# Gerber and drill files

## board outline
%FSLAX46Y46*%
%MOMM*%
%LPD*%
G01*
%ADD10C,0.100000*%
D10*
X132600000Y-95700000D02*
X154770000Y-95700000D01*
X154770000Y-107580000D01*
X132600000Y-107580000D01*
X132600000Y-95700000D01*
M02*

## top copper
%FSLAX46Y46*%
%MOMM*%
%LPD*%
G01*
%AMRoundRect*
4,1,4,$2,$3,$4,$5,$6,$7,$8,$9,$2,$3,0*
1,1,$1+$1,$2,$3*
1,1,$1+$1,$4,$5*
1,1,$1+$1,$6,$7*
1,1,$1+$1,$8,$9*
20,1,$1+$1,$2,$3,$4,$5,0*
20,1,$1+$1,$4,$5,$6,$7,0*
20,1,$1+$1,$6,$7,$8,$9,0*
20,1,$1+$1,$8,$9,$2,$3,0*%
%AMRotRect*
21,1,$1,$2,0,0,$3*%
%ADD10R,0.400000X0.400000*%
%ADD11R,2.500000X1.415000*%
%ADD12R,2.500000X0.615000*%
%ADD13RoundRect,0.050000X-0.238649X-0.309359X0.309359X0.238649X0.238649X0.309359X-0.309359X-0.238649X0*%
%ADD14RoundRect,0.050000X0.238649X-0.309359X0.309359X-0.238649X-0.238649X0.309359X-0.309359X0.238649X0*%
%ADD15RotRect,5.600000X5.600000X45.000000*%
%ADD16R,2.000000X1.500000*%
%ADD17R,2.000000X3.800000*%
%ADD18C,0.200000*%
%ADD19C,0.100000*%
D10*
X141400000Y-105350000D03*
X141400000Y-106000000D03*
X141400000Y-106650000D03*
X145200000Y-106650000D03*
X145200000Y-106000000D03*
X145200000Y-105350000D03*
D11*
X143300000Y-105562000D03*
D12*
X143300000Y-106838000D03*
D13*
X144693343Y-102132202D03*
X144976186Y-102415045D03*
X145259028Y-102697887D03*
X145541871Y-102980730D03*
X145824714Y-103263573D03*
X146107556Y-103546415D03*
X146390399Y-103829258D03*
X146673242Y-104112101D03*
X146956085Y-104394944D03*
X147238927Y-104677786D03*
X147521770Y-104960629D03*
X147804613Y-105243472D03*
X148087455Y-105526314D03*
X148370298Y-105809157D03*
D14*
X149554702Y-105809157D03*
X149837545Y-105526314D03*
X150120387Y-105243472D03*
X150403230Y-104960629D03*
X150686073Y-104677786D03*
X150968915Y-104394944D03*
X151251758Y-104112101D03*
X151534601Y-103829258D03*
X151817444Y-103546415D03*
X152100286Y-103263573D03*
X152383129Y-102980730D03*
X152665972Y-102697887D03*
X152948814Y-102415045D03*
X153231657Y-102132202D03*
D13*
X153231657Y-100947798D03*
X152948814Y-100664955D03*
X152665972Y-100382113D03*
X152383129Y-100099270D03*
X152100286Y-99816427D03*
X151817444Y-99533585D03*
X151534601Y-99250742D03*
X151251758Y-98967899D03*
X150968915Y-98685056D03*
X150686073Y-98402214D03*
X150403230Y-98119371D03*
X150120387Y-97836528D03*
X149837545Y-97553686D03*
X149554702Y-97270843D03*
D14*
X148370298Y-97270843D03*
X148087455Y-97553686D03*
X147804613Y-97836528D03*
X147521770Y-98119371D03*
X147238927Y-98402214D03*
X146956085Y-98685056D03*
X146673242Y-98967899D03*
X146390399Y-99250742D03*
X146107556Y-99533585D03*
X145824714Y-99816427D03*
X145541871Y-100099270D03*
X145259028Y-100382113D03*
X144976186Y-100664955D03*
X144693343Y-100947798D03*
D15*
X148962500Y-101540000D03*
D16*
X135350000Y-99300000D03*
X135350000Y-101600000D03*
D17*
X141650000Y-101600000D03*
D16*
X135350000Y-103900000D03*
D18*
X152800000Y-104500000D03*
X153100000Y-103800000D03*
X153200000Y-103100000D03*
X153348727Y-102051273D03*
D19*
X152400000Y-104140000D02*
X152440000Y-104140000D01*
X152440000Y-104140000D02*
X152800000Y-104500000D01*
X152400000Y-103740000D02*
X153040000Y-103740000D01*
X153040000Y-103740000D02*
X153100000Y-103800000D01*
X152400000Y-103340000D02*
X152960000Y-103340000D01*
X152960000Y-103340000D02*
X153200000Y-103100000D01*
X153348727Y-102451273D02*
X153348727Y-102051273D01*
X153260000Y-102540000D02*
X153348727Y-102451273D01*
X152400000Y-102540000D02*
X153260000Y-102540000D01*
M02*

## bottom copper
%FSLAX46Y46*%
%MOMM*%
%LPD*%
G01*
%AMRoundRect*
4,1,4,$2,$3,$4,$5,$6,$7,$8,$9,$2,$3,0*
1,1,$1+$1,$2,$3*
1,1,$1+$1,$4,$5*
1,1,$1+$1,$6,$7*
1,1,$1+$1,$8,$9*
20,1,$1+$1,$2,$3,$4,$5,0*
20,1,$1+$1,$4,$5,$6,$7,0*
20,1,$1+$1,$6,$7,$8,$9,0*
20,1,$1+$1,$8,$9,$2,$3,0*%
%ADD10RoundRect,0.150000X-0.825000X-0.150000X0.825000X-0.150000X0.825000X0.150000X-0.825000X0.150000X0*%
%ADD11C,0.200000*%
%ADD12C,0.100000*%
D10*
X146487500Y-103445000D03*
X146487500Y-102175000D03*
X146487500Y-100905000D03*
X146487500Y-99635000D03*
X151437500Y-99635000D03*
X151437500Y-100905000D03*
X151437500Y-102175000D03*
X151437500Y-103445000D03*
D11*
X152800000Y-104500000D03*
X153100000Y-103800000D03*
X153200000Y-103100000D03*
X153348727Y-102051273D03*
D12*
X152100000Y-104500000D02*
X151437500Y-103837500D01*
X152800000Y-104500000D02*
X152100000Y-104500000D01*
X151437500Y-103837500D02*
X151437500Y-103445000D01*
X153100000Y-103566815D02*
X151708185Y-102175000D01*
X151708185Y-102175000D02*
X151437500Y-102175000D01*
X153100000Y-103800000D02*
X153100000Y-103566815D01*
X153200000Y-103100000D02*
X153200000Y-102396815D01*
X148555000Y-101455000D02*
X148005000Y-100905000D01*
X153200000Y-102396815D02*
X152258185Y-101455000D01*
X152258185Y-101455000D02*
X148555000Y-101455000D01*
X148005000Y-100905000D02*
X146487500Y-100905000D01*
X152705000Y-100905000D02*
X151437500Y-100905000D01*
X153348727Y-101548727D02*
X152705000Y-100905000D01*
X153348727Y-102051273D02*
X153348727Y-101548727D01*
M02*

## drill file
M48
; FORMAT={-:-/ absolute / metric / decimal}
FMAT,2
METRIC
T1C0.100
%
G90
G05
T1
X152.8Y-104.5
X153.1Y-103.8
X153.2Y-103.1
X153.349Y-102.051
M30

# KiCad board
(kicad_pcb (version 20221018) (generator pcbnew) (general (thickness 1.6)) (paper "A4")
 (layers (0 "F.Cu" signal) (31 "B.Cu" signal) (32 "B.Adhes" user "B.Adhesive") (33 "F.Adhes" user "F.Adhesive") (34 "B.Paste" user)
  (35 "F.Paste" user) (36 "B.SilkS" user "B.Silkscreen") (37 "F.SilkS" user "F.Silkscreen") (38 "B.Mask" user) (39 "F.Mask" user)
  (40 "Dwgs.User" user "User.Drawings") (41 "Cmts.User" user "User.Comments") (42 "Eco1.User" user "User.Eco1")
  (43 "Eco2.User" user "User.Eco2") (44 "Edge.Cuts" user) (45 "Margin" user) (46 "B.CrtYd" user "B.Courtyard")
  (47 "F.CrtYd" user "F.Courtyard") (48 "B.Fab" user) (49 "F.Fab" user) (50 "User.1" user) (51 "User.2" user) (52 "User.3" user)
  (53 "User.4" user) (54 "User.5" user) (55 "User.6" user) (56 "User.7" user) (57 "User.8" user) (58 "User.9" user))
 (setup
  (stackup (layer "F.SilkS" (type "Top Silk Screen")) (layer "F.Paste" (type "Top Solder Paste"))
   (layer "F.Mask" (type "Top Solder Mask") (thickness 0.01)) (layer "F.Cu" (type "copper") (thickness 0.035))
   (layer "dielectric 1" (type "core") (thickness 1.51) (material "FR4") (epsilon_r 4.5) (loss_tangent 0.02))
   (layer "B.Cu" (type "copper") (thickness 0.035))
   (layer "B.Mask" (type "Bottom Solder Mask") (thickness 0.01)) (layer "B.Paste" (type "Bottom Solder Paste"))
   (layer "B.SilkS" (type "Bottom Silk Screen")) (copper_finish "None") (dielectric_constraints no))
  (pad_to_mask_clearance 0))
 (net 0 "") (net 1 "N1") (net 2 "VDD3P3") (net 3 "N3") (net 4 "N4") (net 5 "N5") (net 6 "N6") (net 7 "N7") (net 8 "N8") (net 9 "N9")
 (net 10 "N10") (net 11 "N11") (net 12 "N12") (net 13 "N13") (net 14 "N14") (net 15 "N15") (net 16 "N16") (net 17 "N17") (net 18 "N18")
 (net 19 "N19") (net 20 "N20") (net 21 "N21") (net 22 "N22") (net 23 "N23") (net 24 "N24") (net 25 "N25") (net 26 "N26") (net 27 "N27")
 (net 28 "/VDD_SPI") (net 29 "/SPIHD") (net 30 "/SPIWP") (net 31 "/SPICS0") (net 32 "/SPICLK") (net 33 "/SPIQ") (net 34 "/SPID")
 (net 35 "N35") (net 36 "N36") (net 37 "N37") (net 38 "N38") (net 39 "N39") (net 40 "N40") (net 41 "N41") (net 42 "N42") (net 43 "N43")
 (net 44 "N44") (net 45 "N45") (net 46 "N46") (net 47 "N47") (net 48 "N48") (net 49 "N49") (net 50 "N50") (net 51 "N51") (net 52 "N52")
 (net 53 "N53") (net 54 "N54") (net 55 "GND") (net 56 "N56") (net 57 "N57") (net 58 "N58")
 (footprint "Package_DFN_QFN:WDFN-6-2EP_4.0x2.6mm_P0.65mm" (layer "F.Cu") (at 143.3 106)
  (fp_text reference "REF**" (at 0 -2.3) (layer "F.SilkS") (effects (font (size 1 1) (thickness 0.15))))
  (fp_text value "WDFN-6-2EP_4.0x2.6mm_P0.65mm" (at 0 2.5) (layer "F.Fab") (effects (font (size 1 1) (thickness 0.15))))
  (pad "1" smd rect (at -1.9 -0.65 270) (size 0.4 0.4) (layers "F.Cu" "F.Paste" "F.Mask"))
  (pad "2" smd rect (at -1.9 0 270) (size 0.4 0.4) (layers "F.Cu" "F.Paste" "F.Mask"))
  (pad "3" smd rect (at -1.9 0.65 270) (size 0.4 0.4) (layers "F.Cu" "F.Paste" "F.Mask"))
  (pad "4" smd rect (at 1.9 0.65 270) (size 0.4 0.4) (layers "F.Cu" "F.Paste" "F.Mask"))
  (pad "5" smd rect (at 1.9 0 270) (size 0.4 0.4) (layers "F.Cu" "F.Paste" "F.Mask"))
  (pad "6" smd rect (at 1.9 -0.65 270) (size 0.4 0.4) (layers "F.Cu" "F.Paste" "F.Mask"))
  (pad "7" smd rect (at 0 -0.438 270) (size 1.415 2.5) (layers "F.Cu" "F.Paste" "F.Mask"))
  (pad "8" smd rect (at 0 0.838 270) (size 0.615 2.5) (layers "F.Cu" "F.Paste" "F.Mask")))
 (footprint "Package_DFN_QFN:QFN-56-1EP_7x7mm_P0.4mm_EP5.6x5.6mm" (layer "F.Cu") (at 148.9625 101.54 45)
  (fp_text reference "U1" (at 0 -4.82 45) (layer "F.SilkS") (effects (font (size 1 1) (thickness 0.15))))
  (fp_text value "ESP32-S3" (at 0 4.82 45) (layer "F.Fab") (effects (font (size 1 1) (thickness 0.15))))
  (pad "" smd roundrect (at -2.1 -2.1 45) (size 1.13 1.13) (layers "F.Paste") (roundrect_rratio 0.221239))
  (pad "" smd roundrect (at -2.1 -0.7 45) (size 1.13 1.13) (layers "F.Paste") (roundrect_rratio 0.221239))
  (pad "" smd roundrect (at -2.1 0.7 45) (size 1.13 1.13) (layers "F.Paste") (roundrect_rratio 0.221239))
  (pad "" smd roundrect (at -2.1 2.1 45) (size 1.13 1.13) (layers "F.Paste") (roundrect_rratio 0.221239))
  (pad "" smd roundrect (at -0.7 -2.1 45) (size 1.13 1.13) (layers "F.Paste") (roundrect_rratio 0.221239))
  (pad "" smd roundrect (at -0.7 -0.7 45) (size 1.13 1.13) (layers "F.Paste") (roundrect_rratio 0.221239))
  (pad "" smd roundrect (at -0.7 0.7 45) (size 1.13 1.13) (layers "F.Paste") (roundrect_rratio 0.221239))
  (pad "" smd roundrect (at -0.7 2.1 45) (size 1.13 1.13) (layers "F.Paste") (roundrect_rratio 0.221239))
  (pad "" smd roundrect (at 0.7 -2.1 45) (size 1.13 1.13) (layers "F.Paste") (roundrect_rratio 0.221239))
  (pad "" smd roundrect (at 0.7 -0.7 45) (size 1.13 1.13) (layers "F.Paste") (roundrect_rratio 0.221239))
  (pad "" smd roundrect (at 0.7 0.7 45) (size 1.13 1.13) (layers "F.Paste") (roundrect_rratio 0.221239))
  (pad "" smd roundrect (at 0.7 2.1 45) (size 1.13 1.13) (layers "F.Paste") (roundrect_rratio 0.221239))
  (pad "" smd roundrect (at 2.1 -2.1 45) (size 1.13 1.13) (layers "F.Paste") (roundrect_rratio 0.221239))
  (pad "" smd roundrect (at 2.1 -0.7 45) (size 1.13 1.13) (layers "F.Paste") (roundrect_rratio 0.221239))
  (pad "" smd roundrect (at 2.1 0.7 45) (size 1.13 1.13) (layers "F.Paste") (roundrect_rratio 0.221239))
  (pad "" smd roundrect (at 2.1 2.1 45) (size 1.13 1.13) (layers "F.Paste") (roundrect_rratio 0.221239))
  (pad "1" smd roundrect (at -3.4375 -2.6 45) (size 0.875 0.2) (layers "F.Cu" "F.Paste" "F.Mask") (roundrect_rratio 0.25) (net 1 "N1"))
  (pad "2" smd roundrect (at -3.4375 -2.2 45) (size 0.875 0.2) (layers "F.Cu" "F.Paste" "F.Mask") (roundrect_rratio 0.25) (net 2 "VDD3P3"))
  (pad "3" smd roundrect (at -3.4375 -1.8 45) (size 0.875 0.2) (layers "F.Cu" "F.Paste" "F.Mask") (roundrect_rratio 0.25) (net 2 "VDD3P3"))
  (pad "4" smd roundrect (at -3.4375 -1.4 45) (size 0.875 0.2) (layers "F.Cu" "F.Paste" "F.Mask") (roundrect_rratio 0.25) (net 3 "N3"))
  (pad "5" smd roundrect (at -3.4375 -1 45) (size 0.875 0.2) (layers "F.Cu" "F.Paste" "F.Mask") (roundrect_rratio 0.25) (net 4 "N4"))
  (pad "6" smd roundrect (at -3.4375 -0.6 45) (size 0.875 0.2) (layers "F.Cu" "F.Paste" "F.Mask") (roundrect_rratio 0.25) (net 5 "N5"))
  (pad "7" smd roundrect (at -3.4375 -0.2 45) (size 0.875 0.2) (layers "F.Cu" "F.Paste" "F.Mask") (roundrect_rratio 0.25) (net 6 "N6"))
  (pad "8" smd roundrect (at -3.4375 0.2 45) (size 0.875 0.2) (layers "F.Cu" "F.Paste" "F.Mask") (roundrect_rratio 0.25) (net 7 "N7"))
  (pad "9" smd roundrect (at -3.4375 0.6 45) (size 0.875 0.2) (layers "F.Cu" "F.Paste" "F.Mask") (roundrect_rratio 0.25) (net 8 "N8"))
  (pad "10" smd roundrect (at -3.4375 1 45) (size 0.875 0.2) (layers "F.Cu" "F.Paste" "F.Mask") (roundrect_rratio 0.25) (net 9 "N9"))
  (pad "11" smd roundrect (at -3.4375 1.4 45) (size 0.875 0.2) (layers "F.Cu" "F.Paste" "F.Mask") (roundrect_rratio 0.25) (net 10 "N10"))
  (pad "12" smd roundrect (at -3.4375 1.8 45) (size 0.875 0.2) (layers "F.Cu" "F.Paste" "F.Mask") (roundrect_rratio 0.25) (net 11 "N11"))
  (pad "13" smd roundrect (at -3.4375 2.2 45) (size 0.875 0.2) (layers "F.Cu" "F.Paste" "F.Mask") (roundrect_rratio 0.25) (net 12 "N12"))
  (pad "14" smd roundrect (at -3.4375 2.6 45) (size 0.875 0.2) (layers "F.Cu" "F.Paste" "F.Mask") (roundrect_rratio 0.25) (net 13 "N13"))
  (pad "15" smd roundrect (at -2.6 3.4375 45) (size 0.2 0.875) (layers "F.Cu" "F.Paste" "F.Mask") (roundrect_rratio 0.25) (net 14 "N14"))
  (pad "16" smd roundrect (at -2.2 3.4375 45) (size 0.2 0.875) (layers "F.Cu" "F.Paste" "F.Mask") (roundrect_rratio 0.25) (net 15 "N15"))
  (pad "17" smd roundrect (at -1.8 3.4375 45) (size 0.2 0.875) (layers "F.Cu" "F.Paste" "F.Mask") (roundrect_rratio 0.25) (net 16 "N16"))
  (pad "18" smd roundrect (at -1.4 3.4375 45) (size 0.2 0.875) (layers "F.Cu" "F.Paste" "F.Mask") (roundrect_rratio 0.25) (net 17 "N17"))
  (pad "19" smd roundrect (at -1 3.4375 45) (size 0.2 0.875) (layers "F.Cu" "F.Paste" "F.Mask") (roundrect_rratio 0.25) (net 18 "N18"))
  (pad "20" smd roundrect (at -0.6 3.4375 45) (size 0.2 0.875) (layers "F.Cu" "F.Paste" "F.Mask") (roundrect_rratio 0.25) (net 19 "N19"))
  (pad "21" smd roundrect (at -0.2 3.4375 45) (size 0.2 0.875) (layers "F.Cu" "F.Paste" "F.Mask") (roundrect_rratio 0.25) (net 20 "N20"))
  (pad "22" smd roundrect (at 0.2 3.4375 45) (size 0.2 0.875) (layers "F.Cu" "F.Paste" "F.Mask") (roundrect_rratio 0.25) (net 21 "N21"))
  (pad "23" smd roundrect (at 0.6 3.4375 45) (size 0.2 0.875) (layers "F.Cu" "F.Paste" "F.Mask") (roundrect_rratio 0.25) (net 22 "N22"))
  (pad "24" smd roundrect (at 1 3.4375 45) (size 0.2 0.875) (layers "F.Cu" "F.Paste" "F.Mask") (roundrect_rratio 0.25) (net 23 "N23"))
  (pad "25" smd roundrect (at 1.4 3.4375 45) (size 0.2 0.875) (layers "F.Cu" "F.Paste" "F.Mask") (roundrect_rratio 0.25) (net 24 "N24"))
  (pad "26" smd roundrect (at 1.8 3.4375 45) (size 0.2 0.875) (layers "F.Cu" "F.Paste" "F.Mask") (roundrect_rratio 0.25) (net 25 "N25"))
  (pad "27" smd roundrect (at 2.2 3.4375 45) (size 0.2 0.875) (layers "F.Cu" "F.Paste" "F.Mask") (roundrect_rratio 0.25) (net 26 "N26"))
  (pad "28" smd roundrect (at 2.6 3.4375 45) (size 0.2 0.875) (layers "F.Cu" "F.Paste" "F.Mask") (roundrect_rratio 0.25) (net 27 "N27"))
  (pad "29" smd roundrect (at 3.4375 2.6 45) (size 0.875 0.2) (layers "F.Cu" "F.Paste" "F.Mask") (roundrect_rratio 0.25) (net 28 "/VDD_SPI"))
  (pad "30" smd roundrect (at 3.4375 2.2 45) (size 0.875 0.2) (layers "F.Cu" "F.Paste" "F.Mask") (roundrect_rratio 0.25) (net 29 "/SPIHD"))
  (pad "31" smd roundrect (at 3.4375 1.8 45) (size 0.875 0.2) (layers "F.Cu" "F.Paste" "F.Mask") (roundrect_rratio 0.25) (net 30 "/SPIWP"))
  (pad "32" smd roundrect (at 3.4375 1.4 45) (size 0.875 0.2) (layers "F.Cu" "F.Paste" "F.Mask") (roundrect_rratio 0.25) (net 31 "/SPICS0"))
  (pad "33" smd roundrect (at 3.4375 1 45) (size 0.875 0.2) (layers "F.Cu" "F.Paste" "F.Mask") (roundrect_rratio 0.25) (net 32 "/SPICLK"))
  (pad "34" smd roundrect (at 3.4375 0.6 45) (size 0.875 0.2) (layers "F.Cu" "F.Paste" "F.Mask") (roundrect_rratio 0.25) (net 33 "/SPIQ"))
  (pad "35" smd roundrect (at 3.4375 0.2 45) (size 0.875 0.2) (layers "F.Cu" "F.Paste" "F.Mask") (roundrect_rratio 0.25) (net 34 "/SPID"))
  (pad "36" smd roundrect (at 3.4375 -0.2 45) (size 0.875 0.2) (layers "F.Cu" "F.Paste" "F.Mask") (roundrect_rratio 0.25) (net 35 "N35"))
  (pad "37" smd roundrect (at 3.4375 -0.6 45) (size 0.875 0.2) (layers "F.Cu" "F.Paste" "F.Mask") (roundrect_rratio 0.25) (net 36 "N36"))
  (pad "38" smd roundrect (at 3.4375 -1 45) (size 0.875 0.2) (layers "F.Cu" "F.Paste" "F.Mask") (roundrect_rratio 0.25) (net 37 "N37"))
  (pad "39" smd roundrect (at 3.4375 -1.4 45) (size 0.875 0.2) (layers "F.Cu" "F.Paste" "F.Mask") (roundrect_rratio 0.25) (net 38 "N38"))
  (pad "40" smd roundrect (at 3.4375 -1.8 45) (size 0.875 0.2) (layers "F.Cu" "F.Paste" "F.Mask") (roundrect_rratio 0.25) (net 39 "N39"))
  (pad "41" smd roundrect (at 3.4375 -2.2 45) (size 0.875 0.2) (layers "F.Cu" "F.Paste" "F.Mask") (roundrect_rratio 0.25) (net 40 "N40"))
  (pad "42" smd roundrect (at 3.4375 -2.6 45) (size 0.875 0.2) (layers "F.Cu" "F.Paste" "F.Mask") (roundrect_rratio 0.25) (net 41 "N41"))
  (pad "43" smd roundrect (at 2.6 -3.4375 45) (size 0.2 0.875) (layers "F.Cu" "F.Paste" "F.Mask") (roundrect_rratio 0.25) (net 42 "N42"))
  (pad "44" smd roundrect (at 2.2 -3.4375 45) (size 0.2 0.875) (layers "F.Cu" "F.Paste" "F.Mask") (roundrect_rratio 0.25) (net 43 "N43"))
  (pad "45" smd roundrect (at 1.8 -3.4375 45) (size 0.2 0.875) (layers "F.Cu" "F.Paste" "F.Mask") (roundrect_rratio 0.25) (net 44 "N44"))
  (pad "46" smd roundrect (at 1.4 -3.4375 45) (size 0.2 0.875) (layers "F.Cu" "F.Paste" "F.Mask") (roundrect_rratio 0.25) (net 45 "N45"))
  (pad "47" smd roundrect (at 1 -3.4375 45) (size 0.2 0.875) (layers "F.Cu" "F.Paste" "F.Mask") (roundrect_rratio 0.25) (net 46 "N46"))
  (pad "48" smd roundrect (at 0.6 -3.4375 45) (size 0.2 0.875) (layers "F.Cu" "F.Paste" "F.Mask") (roundrect_rratio 0.25) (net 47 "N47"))
  (pad "49" smd roundrect (at 0.2 -3.4375 45) (size 0.2 0.875) (layers "F.Cu" "F.Paste" "F.Mask") (roundrect_rratio 0.25) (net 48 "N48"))
  (pad "50" smd roundrect (at -0.2 -3.4375 45) (size 0.2 0.875) (layers "F.Cu" "F.Paste" "F.Mask") (roundrect_rratio 0.25) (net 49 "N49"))
  (pad "51" smd roundrect (at -0.6 -3.4375 45) (size 0.2 0.875) (layers "F.Cu" "F.Paste" "F.Mask") (roundrect_rratio 0.25) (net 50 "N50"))
  (pad "52" smd roundrect (at -1 -3.4375 45) (size 0.2 0.875) (layers "F.Cu" "F.Paste" "F.Mask") (roundrect_rratio 0.25) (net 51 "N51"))
  (pad "53" smd roundrect (at -1.4 -3.4375 45) (size 0.2 0.875) (layers "F.Cu" "F.Paste" "F.Mask") (roundrect_rratio 0.25) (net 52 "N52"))
  (pad "54" smd roundrect (at -1.8 -3.4375 45) (size 0.2 0.875) (layers "F.Cu" "F.Paste" "F.Mask") (roundrect_rratio 0.25) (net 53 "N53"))
  (pad "55" smd roundrect (at -2.2 -3.4375 45) (size 0.2 0.875) (layers "F.Cu" "F.Paste" "F.Mask") (roundrect_rratio 0.25) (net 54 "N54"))
  (pad "56" smd roundrect (at -2.6 -3.4375 45) (size 0.2 0.875) (layers "F.Cu" "F.Paste" "F.Mask") (roundrect_rratio 0.25) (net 54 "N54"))
  (pad "57" smd rect (at 0 0 45) (size 5.6 5.6) (layers "F.Cu" "F.Mask") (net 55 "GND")))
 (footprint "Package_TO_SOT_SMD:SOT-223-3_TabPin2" (layer "F.Cu") (at 138.5 101.6)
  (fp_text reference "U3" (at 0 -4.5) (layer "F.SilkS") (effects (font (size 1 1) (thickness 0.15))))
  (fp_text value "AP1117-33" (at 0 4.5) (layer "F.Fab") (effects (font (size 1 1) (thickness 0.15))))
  (pad "1" smd rect (at -3.15 -2.3) (size 2 1.5) (layers "F.Cu" "F.Paste" "F.Mask") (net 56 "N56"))
  (pad "2" smd rect (at -3.15 0) (size 2 1.5) (layers "F.Cu" "F.Paste" "F.Mask") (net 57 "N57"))
  (pad "2" smd rect (at 3.15 0) (size 2 3.8) (layers "F.Cu" "F.Paste" "F.Mask") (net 57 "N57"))
  (pad "3" smd rect (at -3.15 2.3) (size 2 1.5) (layers "F.Cu" "F.Paste" "F.Mask") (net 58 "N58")))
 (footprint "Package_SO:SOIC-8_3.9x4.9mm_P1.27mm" (layer "B.Cu") (at 148.9625 101.54)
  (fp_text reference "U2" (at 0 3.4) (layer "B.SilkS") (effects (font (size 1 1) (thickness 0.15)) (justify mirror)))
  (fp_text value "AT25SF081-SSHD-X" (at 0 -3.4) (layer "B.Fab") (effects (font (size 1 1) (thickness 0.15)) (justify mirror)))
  (pad "1" smd roundrect (at -2.475 1.905) (size 1.95 0.6) (layers "B.Cu" "B.Paste" "B.Mask") (roundrect_rratio 0.25) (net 31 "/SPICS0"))
  (pad "2" smd roundrect (at -2.475 0.635) (size 1.95 0.6) (layers "B.Cu" "B.Paste" "B.Mask") (roundrect_rratio 0.25) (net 33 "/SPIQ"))
  (pad "3" smd roundrect (at -2.475 -0.635) (size 1.95 0.6) (layers "B.Cu" "B.Paste" "B.Mask") (roundrect_rratio 0.25) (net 30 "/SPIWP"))
  (pad "4" smd roundrect (at -2.475 -1.905) (size 1.95 0.6) (layers "B.Cu" "B.Paste" "B.Mask") (roundrect_rratio 0.25) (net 55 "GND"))
  (pad "5" smd roundrect (at 2.475 -1.905) (size 1.95 0.6) (layers "B.Cu" "B.Paste" "B.Mask") (roundrect_rratio 0.25) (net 34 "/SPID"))
  (pad "6" smd roundrect (at 2.475 -0.635) (size 1.95 0.6) (layers "B.Cu" "B.Paste" "B.Mask") (roundrect_rratio 0.25) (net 32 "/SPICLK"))
  (pad "7" smd roundrect (at 2.475 0.635) (size 1.95 0.6) (layers "B.Cu" "B.Paste" "B.Mask") (roundrect_rratio 0.25) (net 29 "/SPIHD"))
  (pad "8" smd roundrect (at 2.475 1.905) (size 1.95 0.6) (layers "B.Cu" "B.Paste" "B.Mask") (roundrect_rratio 0.25) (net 28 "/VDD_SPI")))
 (gr_rect (start 132.6 95.7) (end 154.77 107.58) (stroke (width 0.1) (type default)) (fill none) (layer "Edge.Cuts"))
 (segment (start 152.4 104.14) (end 152.44 104.14) (width 0.1) (layer "F.Cu") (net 28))
 (segment (start 152.44 104.14) (end 152.8 104.5) (width 0.1) (layer "F.Cu") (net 28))
 (via (at 152.8 104.5) (size 0.2) (drill 0.1) (layers "F.Cu" "B.Cu") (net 28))
 (segment (start 152.1 104.5) (end 151.4375 103.8375) (width 0.1) (layer "B.Cu") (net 28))
 (segment (start 152.8 104.5) (end 152.1 104.5) (width 0.1) (layer "B.Cu") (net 28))
 (segment (start 151.4375 103.8375) (end 151.4375 103.445) (width 0.1) (layer "B.Cu") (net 28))
 (segment (start 152.4 103.74) (end 153.04 103.74) (width 0.1) (layer "F.Cu") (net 29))
 (segment (start 153.04 103.74) (end 153.1 103.8) (width 0.1) (layer "F.Cu") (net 29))
 (via (at 153.1 103.8) (size 0.2) (drill 0.1) (layers "F.Cu" "B.Cu") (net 29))
 (segment (start 153.1 103.566815) (end 151.708185 102.175) (width 0.1) (layer "B.Cu") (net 29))
 (segment (start 151.708185 102.175) (end 151.4375 102.175) (width 0.1) (layer "B.Cu") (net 29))
 (segment (start 153.1 103.8) (end 153.1 103.566815) (width 0.1) (layer "B.Cu") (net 29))
 (segment (start 152.4 103.34) (end 152.96 103.34) (width 0.1) (layer "F.Cu") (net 30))
 (segment (start 152.96 103.34) (end 153.2 103.1) (width 0.1) (layer "F.Cu") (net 30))
 (via (at 153.2 103.1) (size 0.2) (drill 0.1) (layers "F.Cu" "B.Cu") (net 30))
 (segment (start 153.2 103.1) (end 153.2 102.396815) (width 0.1) (layer "B.Cu") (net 30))
 (segment (start 148.555 101.455) (end 148.005 100.905) (width 0.1) (layer "B.Cu") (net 30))
 (segment (start 153.2 102.396815) (end 152.258185 101.455) (width 0.1) (layer "B.Cu") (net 30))
 (segment (start 152.258185 101.455) (end 148.555 101.455) (width 0.1) (layer "B.Cu") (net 30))
 (segment (start 148.005 100.905) (end 146.4875 100.905) (width 0.1) (layer "B.Cu") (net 30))
 (segment (start 153.348727 102.451273) (end 153.348727 102.051273) (width 0.1) (layer "F.Cu") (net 32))
 (segment (start 153.26 102.54) (end 153.348727 102.451273) (width 0.1) (layer "F.Cu") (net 32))
 (segment (start 152.4 102.54) (end 153.26 102.54) (width 0.1) (layer "F.Cu") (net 32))
 (via (at 153.348727 102.051273) (size 0.2) (drill 0.1) (layers "F.Cu" "B.Cu") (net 32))
 (segment (start 152.705 100.905) (end 151.4375 100.905) (width 0.1) (layer "B.Cu") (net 32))
 (segment (start 153.348727 101.548727) (end 152.705 100.905) (width 0.1) (layer "B.Cu") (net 32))
 (segment (start 153.348727 102.051273) (end 153.348727 101.548727) (width 0.1) (layer "B.Cu") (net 32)))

